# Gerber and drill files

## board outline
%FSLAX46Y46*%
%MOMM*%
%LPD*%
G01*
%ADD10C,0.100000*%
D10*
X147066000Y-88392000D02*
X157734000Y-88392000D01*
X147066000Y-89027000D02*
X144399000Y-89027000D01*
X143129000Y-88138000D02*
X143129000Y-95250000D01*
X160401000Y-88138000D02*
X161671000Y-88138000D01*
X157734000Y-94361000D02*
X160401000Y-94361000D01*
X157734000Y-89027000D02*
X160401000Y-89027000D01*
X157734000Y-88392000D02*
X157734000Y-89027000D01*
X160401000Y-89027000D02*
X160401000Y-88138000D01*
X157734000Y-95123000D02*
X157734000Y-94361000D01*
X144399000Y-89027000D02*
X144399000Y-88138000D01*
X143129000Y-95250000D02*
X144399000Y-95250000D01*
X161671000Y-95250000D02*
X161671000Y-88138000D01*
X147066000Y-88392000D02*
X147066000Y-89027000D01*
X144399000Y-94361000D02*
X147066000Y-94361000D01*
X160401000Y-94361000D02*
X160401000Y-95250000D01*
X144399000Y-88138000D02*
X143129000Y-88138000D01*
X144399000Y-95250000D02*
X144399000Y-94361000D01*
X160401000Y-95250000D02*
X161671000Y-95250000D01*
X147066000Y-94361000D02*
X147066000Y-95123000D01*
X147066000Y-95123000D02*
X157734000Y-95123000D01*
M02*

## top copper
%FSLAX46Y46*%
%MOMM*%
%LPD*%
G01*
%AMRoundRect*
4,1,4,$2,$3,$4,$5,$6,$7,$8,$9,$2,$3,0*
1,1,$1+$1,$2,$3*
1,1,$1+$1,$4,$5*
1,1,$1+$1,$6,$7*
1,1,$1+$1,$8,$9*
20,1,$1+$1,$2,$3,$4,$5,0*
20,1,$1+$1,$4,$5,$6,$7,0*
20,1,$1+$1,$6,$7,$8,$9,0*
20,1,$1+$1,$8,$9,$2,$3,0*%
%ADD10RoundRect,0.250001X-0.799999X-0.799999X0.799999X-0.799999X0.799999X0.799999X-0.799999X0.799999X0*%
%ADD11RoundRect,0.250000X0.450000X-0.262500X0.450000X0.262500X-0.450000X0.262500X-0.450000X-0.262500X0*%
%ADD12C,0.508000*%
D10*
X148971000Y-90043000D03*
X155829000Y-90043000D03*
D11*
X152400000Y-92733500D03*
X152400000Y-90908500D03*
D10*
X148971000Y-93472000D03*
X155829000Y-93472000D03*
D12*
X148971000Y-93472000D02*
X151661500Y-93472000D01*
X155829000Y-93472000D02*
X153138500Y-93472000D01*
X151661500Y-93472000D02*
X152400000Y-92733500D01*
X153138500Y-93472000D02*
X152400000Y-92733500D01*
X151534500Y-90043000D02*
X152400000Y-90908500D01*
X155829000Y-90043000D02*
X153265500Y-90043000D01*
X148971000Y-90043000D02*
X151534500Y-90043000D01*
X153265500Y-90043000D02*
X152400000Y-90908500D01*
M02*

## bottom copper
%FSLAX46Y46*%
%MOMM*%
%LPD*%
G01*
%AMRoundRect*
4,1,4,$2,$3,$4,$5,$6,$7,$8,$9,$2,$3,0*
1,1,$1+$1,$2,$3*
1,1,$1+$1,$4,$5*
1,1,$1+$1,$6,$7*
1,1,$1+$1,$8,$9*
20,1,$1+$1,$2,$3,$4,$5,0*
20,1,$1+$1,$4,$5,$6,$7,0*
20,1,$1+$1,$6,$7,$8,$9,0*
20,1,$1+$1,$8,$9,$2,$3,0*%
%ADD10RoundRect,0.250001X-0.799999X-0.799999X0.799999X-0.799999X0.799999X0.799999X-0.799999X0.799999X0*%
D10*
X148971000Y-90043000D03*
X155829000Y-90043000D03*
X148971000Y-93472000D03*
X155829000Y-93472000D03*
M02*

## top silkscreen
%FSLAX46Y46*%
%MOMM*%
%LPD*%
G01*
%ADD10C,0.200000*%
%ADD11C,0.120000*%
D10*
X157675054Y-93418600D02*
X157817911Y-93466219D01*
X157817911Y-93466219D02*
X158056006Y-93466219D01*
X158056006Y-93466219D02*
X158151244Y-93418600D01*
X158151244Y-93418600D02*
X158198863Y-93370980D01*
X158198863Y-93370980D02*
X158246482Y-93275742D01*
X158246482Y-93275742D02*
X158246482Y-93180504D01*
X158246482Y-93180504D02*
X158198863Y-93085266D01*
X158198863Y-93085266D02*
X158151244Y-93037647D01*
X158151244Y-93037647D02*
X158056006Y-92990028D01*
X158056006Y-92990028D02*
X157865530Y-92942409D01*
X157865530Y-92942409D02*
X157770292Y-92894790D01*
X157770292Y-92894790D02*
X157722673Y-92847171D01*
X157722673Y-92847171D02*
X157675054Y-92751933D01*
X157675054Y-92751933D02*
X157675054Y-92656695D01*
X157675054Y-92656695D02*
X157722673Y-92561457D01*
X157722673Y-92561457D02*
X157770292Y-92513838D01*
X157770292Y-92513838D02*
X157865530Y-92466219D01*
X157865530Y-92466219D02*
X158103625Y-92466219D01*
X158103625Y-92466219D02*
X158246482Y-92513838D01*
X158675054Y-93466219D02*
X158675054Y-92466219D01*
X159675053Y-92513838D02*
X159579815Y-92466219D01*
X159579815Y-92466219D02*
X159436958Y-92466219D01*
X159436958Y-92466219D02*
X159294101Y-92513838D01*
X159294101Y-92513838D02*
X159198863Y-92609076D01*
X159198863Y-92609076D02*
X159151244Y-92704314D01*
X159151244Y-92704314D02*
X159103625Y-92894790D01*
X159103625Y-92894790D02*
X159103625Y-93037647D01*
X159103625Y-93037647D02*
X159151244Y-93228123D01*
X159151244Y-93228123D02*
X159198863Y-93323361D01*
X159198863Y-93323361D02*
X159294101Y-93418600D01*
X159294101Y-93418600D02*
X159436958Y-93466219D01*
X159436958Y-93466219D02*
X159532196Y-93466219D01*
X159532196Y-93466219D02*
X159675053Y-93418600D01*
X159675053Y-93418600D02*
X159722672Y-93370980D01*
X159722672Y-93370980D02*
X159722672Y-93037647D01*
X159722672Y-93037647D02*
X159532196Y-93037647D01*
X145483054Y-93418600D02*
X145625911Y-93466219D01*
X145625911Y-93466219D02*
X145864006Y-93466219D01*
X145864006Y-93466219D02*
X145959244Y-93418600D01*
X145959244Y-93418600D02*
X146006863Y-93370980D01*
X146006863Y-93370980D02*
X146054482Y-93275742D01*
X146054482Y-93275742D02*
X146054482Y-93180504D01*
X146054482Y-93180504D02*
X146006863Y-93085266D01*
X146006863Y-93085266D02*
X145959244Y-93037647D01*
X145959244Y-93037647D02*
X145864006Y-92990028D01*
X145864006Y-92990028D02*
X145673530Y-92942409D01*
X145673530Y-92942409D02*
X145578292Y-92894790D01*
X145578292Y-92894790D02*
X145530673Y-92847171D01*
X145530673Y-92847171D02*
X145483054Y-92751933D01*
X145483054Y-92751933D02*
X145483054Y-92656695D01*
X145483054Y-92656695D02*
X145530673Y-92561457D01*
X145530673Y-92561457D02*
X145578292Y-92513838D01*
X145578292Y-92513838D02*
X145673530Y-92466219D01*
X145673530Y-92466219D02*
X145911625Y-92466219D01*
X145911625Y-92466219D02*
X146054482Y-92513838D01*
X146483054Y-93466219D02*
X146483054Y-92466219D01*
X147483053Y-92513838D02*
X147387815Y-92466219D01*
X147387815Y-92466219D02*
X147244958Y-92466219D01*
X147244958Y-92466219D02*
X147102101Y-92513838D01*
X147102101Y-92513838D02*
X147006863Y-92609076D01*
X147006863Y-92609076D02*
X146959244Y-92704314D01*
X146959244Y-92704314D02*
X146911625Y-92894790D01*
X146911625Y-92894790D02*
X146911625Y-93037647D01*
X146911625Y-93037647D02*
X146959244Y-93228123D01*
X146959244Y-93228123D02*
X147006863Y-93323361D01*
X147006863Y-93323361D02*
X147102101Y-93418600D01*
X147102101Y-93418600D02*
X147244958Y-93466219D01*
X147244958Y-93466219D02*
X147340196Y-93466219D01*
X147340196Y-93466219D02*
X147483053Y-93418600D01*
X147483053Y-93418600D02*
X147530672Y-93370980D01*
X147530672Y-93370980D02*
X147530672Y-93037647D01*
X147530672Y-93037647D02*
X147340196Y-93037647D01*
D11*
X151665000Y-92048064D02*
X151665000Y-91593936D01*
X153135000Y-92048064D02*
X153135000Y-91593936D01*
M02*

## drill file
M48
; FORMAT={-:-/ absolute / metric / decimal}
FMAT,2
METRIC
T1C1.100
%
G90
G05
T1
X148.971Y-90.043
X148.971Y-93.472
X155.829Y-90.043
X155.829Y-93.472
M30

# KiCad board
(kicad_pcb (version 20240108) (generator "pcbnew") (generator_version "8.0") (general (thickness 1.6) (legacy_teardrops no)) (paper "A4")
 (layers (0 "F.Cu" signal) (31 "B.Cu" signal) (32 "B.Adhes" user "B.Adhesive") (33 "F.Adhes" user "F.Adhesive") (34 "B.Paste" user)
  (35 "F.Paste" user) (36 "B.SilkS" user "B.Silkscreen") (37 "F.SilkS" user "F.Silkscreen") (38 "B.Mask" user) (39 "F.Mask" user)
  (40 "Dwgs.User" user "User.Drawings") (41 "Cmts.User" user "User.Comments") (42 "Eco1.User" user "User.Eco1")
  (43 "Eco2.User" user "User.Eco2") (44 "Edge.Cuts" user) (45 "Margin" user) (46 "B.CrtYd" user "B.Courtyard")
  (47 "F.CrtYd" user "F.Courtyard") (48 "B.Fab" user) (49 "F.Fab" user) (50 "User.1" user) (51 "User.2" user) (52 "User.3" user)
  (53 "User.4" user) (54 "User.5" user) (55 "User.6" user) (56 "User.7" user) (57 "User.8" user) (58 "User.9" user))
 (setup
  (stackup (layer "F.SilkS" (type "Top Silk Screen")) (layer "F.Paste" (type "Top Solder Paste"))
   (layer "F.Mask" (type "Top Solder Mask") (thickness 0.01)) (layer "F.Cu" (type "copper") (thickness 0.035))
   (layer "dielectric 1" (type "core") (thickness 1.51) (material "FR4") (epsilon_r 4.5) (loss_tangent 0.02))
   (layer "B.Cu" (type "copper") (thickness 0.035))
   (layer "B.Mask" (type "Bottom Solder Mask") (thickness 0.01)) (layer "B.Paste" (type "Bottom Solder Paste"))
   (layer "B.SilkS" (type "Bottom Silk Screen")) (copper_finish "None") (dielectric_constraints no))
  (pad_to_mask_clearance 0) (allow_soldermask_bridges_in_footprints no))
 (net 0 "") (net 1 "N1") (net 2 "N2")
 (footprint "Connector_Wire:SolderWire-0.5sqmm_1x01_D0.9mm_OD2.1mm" (layer "F.Cu") (at 148.971 90.043)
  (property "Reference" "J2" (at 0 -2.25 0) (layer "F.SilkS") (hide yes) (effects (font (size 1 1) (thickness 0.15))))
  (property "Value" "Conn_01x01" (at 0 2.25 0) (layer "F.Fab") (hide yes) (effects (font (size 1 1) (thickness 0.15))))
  (pad "1" thru_hole roundrect (at 0 0) (size 2.1 2.1) (drill 1.1) (layers "*.Cu" "*.Mask") (remove_unused_layers no)
   (roundrect_rratio 0.119048) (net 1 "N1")))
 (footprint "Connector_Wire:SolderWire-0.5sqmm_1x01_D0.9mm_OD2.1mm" (layer "F.Cu") (at 155.829 90.043)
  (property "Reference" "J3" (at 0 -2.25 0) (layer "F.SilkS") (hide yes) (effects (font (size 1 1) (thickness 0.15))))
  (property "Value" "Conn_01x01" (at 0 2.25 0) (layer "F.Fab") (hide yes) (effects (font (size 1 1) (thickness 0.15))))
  (pad "1" thru_hole roundrect (at 0 0) (size 2.1 2.1) (drill 1.1) (layers "*.Cu" "*.Mask") (remove_unused_layers no)
   (roundrect_rratio 0.119048) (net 1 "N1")))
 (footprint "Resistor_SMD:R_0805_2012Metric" (layer "F.Cu") (at 152.4 91.821 90)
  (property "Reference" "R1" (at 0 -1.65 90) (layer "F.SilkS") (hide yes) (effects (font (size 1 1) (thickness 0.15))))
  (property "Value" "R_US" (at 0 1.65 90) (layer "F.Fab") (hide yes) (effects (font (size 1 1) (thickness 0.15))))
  (fp_line (start -0.227064 -0.735) (end 0.227064 -0.735) (stroke (width 0.12) (type solid)) (layer "F.SilkS"))
  (fp_line (start -0.227064 0.735) (end 0.227064 0.735) (stroke (width 0.12) (type solid)) (layer "F.SilkS"))
  (pad "1" smd roundrect (at -0.9125 0 90) (size 1.025 1.4) (layers "F.Cu" "F.Paste" "F.Mask") (roundrect_rratio 0.243902) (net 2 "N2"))
  (pad "2" smd roundrect (at 0.9125 0 90) (size 1.025 1.4) (layers "F.Cu" "F.Paste" "F.Mask") (roundrect_rratio 0.243902) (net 1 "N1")))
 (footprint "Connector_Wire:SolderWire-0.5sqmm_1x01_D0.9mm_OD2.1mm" (layer "F.Cu") (at 148.971 93.472)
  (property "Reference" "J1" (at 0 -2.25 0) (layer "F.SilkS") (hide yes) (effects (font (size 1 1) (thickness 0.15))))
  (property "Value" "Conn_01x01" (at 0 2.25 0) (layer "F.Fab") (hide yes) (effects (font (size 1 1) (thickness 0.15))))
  (pad "1" thru_hole roundrect (at 0 0) (size 2.1 2.1) (drill 1.1) (layers "*.Cu" "*.Mask") (remove_unused_layers no)
   (roundrect_rratio 0.119048) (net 2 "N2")))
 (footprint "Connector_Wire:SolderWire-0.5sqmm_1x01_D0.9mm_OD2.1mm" (layer "F.Cu") (at 155.829 93.472)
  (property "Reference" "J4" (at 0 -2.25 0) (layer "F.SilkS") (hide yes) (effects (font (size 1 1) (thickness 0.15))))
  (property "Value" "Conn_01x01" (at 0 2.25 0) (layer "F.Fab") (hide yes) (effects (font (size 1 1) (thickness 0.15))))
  (pad "1" thru_hole roundrect (at 0 0) (size 2.1 2.1) (drill 1.1) (layers "*.Cu" "*.Mask") (remove_unused_layers no)
   (roundrect_rratio 0.119048) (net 2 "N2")))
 (gr_line (start 147.066 88.392) (end 157.734 88.392) (stroke (width 0.1) (type default)) (layer "Edge.Cuts"))
 (gr_line (start 147.066 89.027) (end 144.399 89.027) (stroke (width 0.1) (type default)) (layer "Edge.Cuts"))
 (gr_line (start 143.129 88.138) (end 143.129 95.25) (stroke (width 0.1) (type default)) (layer "Edge.Cuts"))
 (gr_line (start 160.401 88.138) (end 161.671 88.138) (stroke (width 0.1) (type default)) (layer "Edge.Cuts"))
 (gr_line (start 157.734 94.361) (end 160.401 94.361) (stroke (width 0.1) (type default)) (layer "Edge.Cuts"))
 (gr_line (start 157.734 89.027) (end 160.401 89.027) (stroke (width 0.1) (type default)) (layer "Edge.Cuts"))
 (gr_line (start 157.734 88.392) (end 157.734 89.027) (stroke (width 0.1) (type default)) (layer "Edge.Cuts"))
 (gr_line (start 160.401 89.027) (end 160.401 88.138) (stroke (width 0.1) (type default)) (layer "Edge.Cuts"))
 (gr_line (start 157.734 95.123) (end 157.734 94.361) (stroke (width 0.1) (type default)) (layer "Edge.Cuts"))
 (gr_line (start 144.399 89.027) (end 144.399 88.138) (stroke (width 0.1) (type default)) (layer "Edge.Cuts"))
 (gr_line (start 143.129 95.25) (end 144.399 95.25) (stroke (width 0.1) (type default)) (layer "Edge.Cuts"))
 (gr_line (start 161.671 95.25) (end 161.671 88.138) (stroke (width 0.1) (type default)) (layer "Edge.Cuts"))
 (gr_line (start 147.066 88.392) (end 147.066 89.027) (stroke (width 0.1) (type default)) (layer "Edge.Cuts"))
 (gr_line (start 144.399 94.361) (end 147.066 94.361) (stroke (width 0.1) (type default)) (layer "Edge.Cuts"))
 (gr_line (start 160.401 94.361) (end 160.401 95.25) (stroke (width 0.1) (type default)) (layer "Edge.Cuts"))
 (gr_line (start 144.399 88.138) (end 143.129 88.138) (stroke (width 0.1) (type default)) (layer "Edge.Cuts"))
 (gr_line (start 144.399 95.25) (end 144.399 94.361) (stroke (width 0.1) (type default)) (layer "Edge.Cuts"))
 (gr_line (start 160.401 95.25) (end 161.671 95.25) (stroke (width 0.1) (type default)) (layer "Edge.Cuts"))
 (gr_line (start 147.066 94.361) (end 147.066 95.123) (stroke (width 0.1) (type default)) (layer "Edge.Cuts"))
 (gr_line (start 147.066 95.123) (end 157.734 95.123) (stroke (width 0.1) (type default)) (layer "Edge.Cuts"))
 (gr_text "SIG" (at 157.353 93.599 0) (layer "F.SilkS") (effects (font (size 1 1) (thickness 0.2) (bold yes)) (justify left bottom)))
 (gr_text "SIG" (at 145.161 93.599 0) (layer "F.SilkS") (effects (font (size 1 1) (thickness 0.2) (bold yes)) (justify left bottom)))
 (segment (start 148.971 93.472) (end 151.6615 93.472) (width 0.508) (layer "F.Cu") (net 2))
 (segment (start 155.829 93.472) (end 153.1385 93.472) (width 0.508) (layer "F.Cu") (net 2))
 (segment (start 151.6615 93.472) (end 152.4 92.7335) (width 0.508) (layer "F.Cu") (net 2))
 (segment (start 153.1385 93.472) (end 152.4 92.7335) (width 0.508) (layer "F.Cu") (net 2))
 (segment (start 151.5345 90.043) (end 152.4 90.9085) (width 0.508) (layer "F.Cu") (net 1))
 (segment (start 155.829 90.043) (end 153.2655 90.043) (width 0.508) (layer "F.Cu") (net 1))
 (segment (start 148.971 90.043) (end 151.5345 90.043) (width 0.508) (layer "F.Cu") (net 1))
 (segment (start 153.2655 90.043) (end 152.4 90.9085) (width 0.508) (layer "F.Cu") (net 1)))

